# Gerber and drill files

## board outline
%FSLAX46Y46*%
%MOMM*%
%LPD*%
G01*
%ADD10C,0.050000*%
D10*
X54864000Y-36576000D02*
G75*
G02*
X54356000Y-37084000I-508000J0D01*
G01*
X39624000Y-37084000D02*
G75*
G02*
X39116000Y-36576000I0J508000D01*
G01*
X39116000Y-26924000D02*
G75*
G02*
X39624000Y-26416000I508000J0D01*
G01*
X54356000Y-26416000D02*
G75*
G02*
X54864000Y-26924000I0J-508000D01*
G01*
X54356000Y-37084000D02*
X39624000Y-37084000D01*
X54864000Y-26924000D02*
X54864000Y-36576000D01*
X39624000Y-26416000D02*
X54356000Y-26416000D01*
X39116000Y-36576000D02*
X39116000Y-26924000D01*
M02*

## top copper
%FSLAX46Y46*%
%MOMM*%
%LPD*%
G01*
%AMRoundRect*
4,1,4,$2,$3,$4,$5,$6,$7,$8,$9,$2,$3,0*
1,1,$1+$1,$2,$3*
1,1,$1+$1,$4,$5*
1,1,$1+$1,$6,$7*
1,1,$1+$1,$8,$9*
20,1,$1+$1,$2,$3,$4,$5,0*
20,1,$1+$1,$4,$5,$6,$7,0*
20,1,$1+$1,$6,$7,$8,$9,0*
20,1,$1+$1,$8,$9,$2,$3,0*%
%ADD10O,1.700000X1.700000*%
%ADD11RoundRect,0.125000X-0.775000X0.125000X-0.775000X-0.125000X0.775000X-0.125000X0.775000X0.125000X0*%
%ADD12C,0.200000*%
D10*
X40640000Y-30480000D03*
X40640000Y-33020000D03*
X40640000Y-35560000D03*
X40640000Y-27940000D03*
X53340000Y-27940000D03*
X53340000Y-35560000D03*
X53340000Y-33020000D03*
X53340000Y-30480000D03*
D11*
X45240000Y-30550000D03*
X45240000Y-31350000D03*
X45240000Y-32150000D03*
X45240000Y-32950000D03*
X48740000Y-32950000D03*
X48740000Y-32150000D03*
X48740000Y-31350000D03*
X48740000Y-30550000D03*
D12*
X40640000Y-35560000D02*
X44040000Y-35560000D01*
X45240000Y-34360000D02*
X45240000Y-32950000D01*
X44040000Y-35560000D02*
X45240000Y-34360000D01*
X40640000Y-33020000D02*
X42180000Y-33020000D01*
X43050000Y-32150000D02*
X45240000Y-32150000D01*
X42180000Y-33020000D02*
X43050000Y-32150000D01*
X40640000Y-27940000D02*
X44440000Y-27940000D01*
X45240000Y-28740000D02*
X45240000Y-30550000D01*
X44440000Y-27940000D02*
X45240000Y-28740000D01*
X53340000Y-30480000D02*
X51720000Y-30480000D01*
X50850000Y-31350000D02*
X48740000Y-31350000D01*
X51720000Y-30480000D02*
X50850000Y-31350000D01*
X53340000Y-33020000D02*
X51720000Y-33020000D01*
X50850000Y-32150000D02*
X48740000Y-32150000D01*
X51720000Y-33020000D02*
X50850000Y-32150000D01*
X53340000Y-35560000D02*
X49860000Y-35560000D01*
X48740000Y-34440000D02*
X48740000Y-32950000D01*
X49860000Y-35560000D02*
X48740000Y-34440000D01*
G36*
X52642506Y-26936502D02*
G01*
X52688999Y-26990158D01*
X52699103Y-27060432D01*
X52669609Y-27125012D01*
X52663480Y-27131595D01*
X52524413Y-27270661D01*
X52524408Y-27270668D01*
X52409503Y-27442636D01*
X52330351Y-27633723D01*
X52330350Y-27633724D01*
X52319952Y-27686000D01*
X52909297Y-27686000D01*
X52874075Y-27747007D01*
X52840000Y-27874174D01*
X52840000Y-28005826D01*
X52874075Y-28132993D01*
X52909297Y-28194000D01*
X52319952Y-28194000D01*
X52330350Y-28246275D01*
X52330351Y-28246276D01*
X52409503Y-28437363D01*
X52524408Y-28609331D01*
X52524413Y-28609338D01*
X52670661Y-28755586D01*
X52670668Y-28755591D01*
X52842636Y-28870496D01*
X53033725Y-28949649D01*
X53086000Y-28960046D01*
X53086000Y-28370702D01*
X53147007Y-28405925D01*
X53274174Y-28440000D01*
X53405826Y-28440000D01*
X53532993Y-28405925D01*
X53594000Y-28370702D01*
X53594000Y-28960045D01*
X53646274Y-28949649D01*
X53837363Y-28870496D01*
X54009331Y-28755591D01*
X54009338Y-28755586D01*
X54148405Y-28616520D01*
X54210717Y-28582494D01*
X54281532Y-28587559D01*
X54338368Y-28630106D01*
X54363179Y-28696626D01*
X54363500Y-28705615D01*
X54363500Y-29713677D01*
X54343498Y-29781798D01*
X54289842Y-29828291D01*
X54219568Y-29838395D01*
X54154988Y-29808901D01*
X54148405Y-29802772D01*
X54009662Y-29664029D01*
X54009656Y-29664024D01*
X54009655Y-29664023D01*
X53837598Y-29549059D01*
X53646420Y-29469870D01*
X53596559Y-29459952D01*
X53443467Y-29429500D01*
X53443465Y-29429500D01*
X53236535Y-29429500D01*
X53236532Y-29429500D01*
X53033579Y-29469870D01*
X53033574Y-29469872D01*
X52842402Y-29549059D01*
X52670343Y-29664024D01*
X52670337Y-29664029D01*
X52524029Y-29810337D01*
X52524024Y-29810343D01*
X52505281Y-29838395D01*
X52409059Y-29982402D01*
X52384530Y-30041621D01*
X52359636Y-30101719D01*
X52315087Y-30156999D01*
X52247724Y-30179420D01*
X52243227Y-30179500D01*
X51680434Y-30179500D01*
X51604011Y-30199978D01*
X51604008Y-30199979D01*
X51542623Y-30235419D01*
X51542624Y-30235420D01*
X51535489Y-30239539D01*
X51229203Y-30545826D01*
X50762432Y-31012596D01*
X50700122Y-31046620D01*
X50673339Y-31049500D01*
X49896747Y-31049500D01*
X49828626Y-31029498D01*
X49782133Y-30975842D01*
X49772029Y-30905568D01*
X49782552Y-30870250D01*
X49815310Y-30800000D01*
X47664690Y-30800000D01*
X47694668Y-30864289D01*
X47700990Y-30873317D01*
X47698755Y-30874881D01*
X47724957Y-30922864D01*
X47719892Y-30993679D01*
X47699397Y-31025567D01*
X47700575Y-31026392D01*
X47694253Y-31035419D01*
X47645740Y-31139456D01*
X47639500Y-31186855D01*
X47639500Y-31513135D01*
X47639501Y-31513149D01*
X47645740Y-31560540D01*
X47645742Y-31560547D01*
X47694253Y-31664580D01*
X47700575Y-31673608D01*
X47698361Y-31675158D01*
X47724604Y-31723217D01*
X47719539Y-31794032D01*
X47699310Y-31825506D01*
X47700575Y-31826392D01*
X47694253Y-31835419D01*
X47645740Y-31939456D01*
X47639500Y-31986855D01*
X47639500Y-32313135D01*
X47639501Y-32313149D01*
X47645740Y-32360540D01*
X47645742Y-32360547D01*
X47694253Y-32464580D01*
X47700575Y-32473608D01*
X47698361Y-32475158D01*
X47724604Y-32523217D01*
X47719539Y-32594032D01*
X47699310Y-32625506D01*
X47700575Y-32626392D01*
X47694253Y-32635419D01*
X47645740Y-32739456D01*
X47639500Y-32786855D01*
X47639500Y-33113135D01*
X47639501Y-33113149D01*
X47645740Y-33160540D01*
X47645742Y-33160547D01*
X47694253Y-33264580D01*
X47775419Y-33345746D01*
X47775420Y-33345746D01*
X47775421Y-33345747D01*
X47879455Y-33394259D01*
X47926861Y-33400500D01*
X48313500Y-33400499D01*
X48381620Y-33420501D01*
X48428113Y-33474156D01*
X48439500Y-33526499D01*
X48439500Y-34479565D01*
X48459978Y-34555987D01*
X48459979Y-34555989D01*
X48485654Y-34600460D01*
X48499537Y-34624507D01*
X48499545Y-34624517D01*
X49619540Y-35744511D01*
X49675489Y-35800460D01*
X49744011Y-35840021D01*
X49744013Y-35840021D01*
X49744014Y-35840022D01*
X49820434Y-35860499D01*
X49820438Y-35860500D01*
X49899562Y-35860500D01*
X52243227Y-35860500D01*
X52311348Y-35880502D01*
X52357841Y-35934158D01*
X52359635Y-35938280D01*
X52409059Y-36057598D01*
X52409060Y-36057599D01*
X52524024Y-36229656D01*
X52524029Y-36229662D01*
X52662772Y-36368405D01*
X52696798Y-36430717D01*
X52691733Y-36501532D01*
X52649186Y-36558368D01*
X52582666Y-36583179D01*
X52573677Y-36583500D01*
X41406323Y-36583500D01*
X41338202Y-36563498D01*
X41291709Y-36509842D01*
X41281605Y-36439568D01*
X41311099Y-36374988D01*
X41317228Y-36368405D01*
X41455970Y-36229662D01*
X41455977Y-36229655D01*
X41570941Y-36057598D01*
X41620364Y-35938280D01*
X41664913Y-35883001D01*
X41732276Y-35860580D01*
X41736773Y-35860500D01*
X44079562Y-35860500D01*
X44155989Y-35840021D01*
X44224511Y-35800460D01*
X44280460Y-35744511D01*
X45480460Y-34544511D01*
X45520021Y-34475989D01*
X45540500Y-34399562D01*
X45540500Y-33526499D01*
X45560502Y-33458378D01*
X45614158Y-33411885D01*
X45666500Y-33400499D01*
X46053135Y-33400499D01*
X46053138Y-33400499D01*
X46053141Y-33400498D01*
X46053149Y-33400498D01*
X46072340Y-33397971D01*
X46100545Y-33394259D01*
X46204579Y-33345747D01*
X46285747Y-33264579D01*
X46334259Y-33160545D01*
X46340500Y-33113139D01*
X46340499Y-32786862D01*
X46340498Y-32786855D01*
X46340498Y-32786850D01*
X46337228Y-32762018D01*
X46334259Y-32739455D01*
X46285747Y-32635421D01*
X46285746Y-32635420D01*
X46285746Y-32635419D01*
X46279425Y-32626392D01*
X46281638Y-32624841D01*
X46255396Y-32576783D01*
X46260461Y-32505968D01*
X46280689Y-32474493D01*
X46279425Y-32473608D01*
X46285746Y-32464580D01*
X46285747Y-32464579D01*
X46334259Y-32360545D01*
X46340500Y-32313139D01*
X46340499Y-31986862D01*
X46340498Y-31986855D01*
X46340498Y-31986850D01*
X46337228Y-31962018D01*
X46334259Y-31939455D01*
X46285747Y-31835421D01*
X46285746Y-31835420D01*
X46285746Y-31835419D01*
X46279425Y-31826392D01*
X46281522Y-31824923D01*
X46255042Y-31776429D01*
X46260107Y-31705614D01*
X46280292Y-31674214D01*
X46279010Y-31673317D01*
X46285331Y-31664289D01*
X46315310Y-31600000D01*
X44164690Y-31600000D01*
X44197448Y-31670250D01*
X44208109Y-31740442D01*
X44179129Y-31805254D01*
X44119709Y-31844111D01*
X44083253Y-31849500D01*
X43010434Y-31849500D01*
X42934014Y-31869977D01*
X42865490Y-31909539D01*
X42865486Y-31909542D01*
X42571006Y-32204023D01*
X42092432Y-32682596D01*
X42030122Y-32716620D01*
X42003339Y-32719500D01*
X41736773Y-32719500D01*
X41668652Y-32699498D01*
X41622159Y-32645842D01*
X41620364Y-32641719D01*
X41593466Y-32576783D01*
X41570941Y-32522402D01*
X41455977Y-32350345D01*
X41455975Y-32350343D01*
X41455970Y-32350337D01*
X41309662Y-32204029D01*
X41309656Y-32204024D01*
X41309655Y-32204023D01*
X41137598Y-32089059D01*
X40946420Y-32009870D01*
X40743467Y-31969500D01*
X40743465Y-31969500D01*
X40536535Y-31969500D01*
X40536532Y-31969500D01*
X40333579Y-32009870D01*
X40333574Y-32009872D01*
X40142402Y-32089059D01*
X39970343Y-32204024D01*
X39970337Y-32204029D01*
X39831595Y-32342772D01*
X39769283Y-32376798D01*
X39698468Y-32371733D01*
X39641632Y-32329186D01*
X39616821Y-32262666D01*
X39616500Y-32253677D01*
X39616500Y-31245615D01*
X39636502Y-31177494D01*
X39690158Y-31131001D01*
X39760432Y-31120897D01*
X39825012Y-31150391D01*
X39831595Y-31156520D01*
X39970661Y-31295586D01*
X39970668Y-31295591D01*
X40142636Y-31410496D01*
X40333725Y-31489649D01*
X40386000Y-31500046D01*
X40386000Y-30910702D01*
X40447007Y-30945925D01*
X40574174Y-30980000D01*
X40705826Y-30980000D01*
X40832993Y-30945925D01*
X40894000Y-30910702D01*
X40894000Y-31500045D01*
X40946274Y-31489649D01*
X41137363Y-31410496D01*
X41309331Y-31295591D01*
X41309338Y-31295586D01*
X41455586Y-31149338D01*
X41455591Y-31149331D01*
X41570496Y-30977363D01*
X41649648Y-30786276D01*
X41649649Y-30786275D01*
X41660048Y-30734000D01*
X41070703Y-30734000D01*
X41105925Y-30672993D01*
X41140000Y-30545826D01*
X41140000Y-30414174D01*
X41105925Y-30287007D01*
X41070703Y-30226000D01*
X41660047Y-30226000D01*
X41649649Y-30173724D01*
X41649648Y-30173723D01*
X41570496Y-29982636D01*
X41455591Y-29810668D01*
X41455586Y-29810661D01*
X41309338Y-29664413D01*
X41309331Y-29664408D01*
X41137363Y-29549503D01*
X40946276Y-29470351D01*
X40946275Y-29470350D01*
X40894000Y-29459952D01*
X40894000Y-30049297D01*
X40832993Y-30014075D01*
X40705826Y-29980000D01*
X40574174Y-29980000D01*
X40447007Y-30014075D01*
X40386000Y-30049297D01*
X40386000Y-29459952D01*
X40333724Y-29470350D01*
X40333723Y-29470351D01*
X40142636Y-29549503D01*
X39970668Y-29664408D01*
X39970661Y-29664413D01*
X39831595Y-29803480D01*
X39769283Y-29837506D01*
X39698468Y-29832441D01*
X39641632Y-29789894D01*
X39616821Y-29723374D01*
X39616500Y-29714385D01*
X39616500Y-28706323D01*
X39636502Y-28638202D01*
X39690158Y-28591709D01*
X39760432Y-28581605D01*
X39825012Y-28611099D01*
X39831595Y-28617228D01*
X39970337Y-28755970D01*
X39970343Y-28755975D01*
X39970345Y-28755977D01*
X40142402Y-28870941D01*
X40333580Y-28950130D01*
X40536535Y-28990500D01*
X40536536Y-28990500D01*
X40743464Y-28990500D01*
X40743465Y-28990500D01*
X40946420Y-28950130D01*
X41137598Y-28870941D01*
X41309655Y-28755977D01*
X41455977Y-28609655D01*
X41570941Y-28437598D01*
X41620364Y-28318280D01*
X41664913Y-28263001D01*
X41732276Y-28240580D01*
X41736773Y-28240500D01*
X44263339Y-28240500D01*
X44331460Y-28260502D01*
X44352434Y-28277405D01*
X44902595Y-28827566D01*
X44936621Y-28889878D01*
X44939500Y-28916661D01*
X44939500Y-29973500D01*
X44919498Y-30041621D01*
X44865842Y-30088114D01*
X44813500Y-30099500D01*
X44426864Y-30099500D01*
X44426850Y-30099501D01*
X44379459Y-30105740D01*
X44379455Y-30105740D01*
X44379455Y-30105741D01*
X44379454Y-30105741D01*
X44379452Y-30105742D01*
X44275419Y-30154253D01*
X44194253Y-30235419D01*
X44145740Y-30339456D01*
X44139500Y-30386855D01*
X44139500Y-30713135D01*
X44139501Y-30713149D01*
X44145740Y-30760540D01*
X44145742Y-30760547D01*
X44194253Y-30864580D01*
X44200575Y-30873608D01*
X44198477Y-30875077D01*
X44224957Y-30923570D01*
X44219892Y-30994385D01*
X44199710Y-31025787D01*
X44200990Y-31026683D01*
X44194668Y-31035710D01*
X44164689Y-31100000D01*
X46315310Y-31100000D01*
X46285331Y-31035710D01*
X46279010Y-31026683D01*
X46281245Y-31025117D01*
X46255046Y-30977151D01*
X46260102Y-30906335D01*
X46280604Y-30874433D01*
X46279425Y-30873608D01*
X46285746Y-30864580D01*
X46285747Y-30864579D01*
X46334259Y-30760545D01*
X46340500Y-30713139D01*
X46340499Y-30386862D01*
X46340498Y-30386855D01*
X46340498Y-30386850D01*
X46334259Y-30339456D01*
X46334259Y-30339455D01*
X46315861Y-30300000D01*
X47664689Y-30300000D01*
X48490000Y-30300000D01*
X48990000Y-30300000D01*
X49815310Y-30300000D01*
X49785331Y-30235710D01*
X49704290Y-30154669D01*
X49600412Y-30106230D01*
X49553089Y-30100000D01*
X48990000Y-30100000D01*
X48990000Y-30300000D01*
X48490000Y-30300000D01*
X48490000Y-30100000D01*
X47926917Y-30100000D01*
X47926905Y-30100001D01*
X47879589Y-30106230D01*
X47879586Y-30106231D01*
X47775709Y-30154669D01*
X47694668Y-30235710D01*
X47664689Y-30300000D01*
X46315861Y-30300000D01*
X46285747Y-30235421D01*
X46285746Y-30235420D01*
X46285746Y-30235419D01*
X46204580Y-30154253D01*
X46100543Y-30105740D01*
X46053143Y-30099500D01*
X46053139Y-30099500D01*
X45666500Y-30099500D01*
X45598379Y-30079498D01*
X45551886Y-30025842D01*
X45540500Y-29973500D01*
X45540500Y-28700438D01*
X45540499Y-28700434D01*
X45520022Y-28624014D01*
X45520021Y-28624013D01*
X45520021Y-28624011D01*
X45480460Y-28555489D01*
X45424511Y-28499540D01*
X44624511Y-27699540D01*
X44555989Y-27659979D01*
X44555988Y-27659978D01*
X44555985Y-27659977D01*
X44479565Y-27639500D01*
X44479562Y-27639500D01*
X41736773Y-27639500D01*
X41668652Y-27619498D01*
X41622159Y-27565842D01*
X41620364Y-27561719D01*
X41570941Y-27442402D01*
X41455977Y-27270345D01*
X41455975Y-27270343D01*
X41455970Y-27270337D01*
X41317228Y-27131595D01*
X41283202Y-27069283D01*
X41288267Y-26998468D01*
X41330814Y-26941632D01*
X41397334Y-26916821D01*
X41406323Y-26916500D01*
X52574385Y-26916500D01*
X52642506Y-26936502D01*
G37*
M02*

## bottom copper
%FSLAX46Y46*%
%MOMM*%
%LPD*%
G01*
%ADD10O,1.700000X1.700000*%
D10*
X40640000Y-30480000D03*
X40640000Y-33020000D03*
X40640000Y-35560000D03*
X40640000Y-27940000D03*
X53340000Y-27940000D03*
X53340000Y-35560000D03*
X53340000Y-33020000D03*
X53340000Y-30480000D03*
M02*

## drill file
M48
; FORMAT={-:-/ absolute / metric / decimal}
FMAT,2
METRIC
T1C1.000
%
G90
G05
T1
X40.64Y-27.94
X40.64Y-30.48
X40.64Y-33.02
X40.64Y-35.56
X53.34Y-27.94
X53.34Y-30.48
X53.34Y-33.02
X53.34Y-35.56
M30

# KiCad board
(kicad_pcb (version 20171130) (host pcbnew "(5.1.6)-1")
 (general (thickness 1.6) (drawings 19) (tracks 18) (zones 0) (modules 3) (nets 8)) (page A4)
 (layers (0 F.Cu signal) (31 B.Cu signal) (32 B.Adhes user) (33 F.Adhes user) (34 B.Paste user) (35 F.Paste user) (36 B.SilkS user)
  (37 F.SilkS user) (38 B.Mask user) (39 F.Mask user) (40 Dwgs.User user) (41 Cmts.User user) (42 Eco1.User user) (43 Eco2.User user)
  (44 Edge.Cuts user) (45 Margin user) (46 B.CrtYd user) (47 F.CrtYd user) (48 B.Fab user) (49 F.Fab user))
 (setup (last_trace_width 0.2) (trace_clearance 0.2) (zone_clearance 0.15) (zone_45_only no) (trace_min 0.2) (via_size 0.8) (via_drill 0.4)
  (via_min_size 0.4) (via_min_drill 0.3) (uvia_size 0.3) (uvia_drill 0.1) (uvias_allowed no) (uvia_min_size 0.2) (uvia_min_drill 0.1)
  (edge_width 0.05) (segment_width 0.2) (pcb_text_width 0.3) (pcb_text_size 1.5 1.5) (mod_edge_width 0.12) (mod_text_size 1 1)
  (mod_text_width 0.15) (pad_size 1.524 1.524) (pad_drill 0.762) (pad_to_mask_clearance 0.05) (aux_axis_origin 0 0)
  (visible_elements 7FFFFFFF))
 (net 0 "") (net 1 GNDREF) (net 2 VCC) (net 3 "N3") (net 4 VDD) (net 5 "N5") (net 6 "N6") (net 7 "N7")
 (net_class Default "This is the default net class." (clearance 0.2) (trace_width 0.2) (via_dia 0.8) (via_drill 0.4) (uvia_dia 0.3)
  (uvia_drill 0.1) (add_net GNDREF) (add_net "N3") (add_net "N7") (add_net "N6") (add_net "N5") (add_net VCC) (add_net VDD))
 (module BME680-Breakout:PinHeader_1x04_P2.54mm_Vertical (layer F.Cu) (at 40.64 31.75)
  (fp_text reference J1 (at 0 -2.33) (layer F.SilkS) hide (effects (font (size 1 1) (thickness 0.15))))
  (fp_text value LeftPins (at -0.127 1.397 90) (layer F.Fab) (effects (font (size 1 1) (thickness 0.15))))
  (pad 2 thru_hole oval (at 0 -1.27) (size 1.7 1.7) (drill 1) (layers *.Cu *.Mask) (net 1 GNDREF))
  (pad 3 thru_hole oval (at 0 1.27) (size 1.7 1.7) (drill 1) (layers *.Cu *.Mask) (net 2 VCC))
  (pad 4 thru_hole oval (at 0 3.81) (size 1.7 1.7) (drill 1) (layers *.Cu *.Mask) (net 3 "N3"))
  (pad 1 thru_hole oval (at 0 -3.81) (size 1.7 1.7) (drill 1) (layers *.Cu *.Mask) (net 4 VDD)))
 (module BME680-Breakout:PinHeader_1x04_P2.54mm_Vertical (layer F.Cu) (at 53.34 31.75)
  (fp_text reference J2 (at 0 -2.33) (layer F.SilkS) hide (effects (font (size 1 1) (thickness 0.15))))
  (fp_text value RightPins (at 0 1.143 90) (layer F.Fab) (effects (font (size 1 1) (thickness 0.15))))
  (pad 1 thru_hole oval (at 0 -3.81) (size 1.7 1.7) (drill 1) (layers *.Cu *.Mask) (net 1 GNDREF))
  (pad 4 thru_hole oval (at 0 3.81) (size 1.7 1.7) (drill 1) (layers *.Cu *.Mask) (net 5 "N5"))
  (pad 3 thru_hole oval (at 0 1.27) (size 1.7 1.7) (drill 1) (layers *.Cu *.Mask) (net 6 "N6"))
  (pad 2 thru_hole oval (at 0 -1.27) (size 1.7 1.7) (drill 1) (layers *.Cu *.Mask) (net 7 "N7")))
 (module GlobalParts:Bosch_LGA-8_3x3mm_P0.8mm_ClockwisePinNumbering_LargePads (layer F.Cu) (at 46.99 31.75)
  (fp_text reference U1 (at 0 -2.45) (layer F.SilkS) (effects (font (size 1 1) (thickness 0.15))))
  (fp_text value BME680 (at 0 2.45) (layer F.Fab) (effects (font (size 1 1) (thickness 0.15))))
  (pad 8 smd roundrect (at -1.75 -1.2 270) (size 0.5 1.8) (layers F.Cu F.Paste F.Mask) (roundrect_rratio 0.25) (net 4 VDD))
  (pad 7 smd roundrect (at -1.75 -0.4 270) (size 0.5 1.8) (layers F.Cu F.Paste F.Mask) (roundrect_rratio 0.25) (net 1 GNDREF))
  (pad 6 smd roundrect (at -1.75 0.4 270) (size 0.5 1.8) (layers F.Cu F.Paste F.Mask) (roundrect_rratio 0.25) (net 2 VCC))
  (pad 5 smd roundrect (at -1.75 1.2 270) (size 0.5 1.8) (layers F.Cu F.Paste F.Mask) (roundrect_rratio 0.25) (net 3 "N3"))
  (pad 4 smd roundrect (at 1.75 1.2 270) (size 0.5 1.8) (layers F.Cu F.Paste F.Mask) (roundrect_rratio 0.25) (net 5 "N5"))
  (pad 3 smd roundrect (at 1.75 0.4 270) (size 0.5 1.8) (layers F.Cu F.Paste F.Mask) (roundrect_rratio 0.25) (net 6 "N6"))
  (pad 2 smd roundrect (at 1.75 -0.4 270) (size 0.5 1.8) (layers F.Cu F.Paste F.Mask) (roundrect_rratio 0.25) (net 7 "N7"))
  (pad 1 smd roundrect (at 1.75 -1.2 270) (size 0.5 1.8) (layers F.Cu F.Paste F.Mask) (roundrect_rratio 0.25) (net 1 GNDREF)))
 (gr_arc (start 54.356 36.576) (end 54.356 37.084) (angle -90) (layer Edge.Cuts) (width 0.05))
 (gr_arc (start 39.624 36.576) (end 39.116 36.576) (angle -90) (layer Edge.Cuts) (width 0.05))
 (gr_arc (start 39.624 26.924) (end 39.624 26.416) (angle -90) (layer Edge.Cuts) (width 0.05))
 (gr_arc (start 54.356 26.924) (end 54.864 26.924) (angle -90) (layer Edge.Cuts) (width 0.05))
 (gr_line (start 54.356 37.084) (end 39.624 37.084) (layer Edge.Cuts) (width 0.05))
 (gr_line (start 54.864 26.924) (end 54.864 36.576) (layer Edge.Cuts) (width 0.05))
 (gr_line (start 39.624 26.416) (end 54.356 26.416) (layer Edge.Cuts) (width 0.05))
 (gr_line (start 39.116 36.576) (end 39.116 26.924) (layer Edge.Cuts) (width 0.05))
 (segment (start 40.64 35.56) (end 44.04 35.56) (width 0.2) (layer F.Cu) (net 3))
 (segment (start 45.24 34.36) (end 45.24 32.95) (width 0.2) (layer F.Cu) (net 3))
 (segment (start 44.04 35.56) (end 45.24 34.36) (width 0.2) (layer F.Cu) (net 3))
 (segment (start 40.64 33.02) (end 42.18 33.02) (width 0.2) (layer F.Cu) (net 2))
 (segment (start 43.05 32.15) (end 45.24 32.15) (width 0.2) (layer F.Cu) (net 2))
 (segment (start 42.18 33.02) (end 43.05 32.15) (width 0.2) (layer F.Cu) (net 2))
 (segment (start 40.64 27.94) (end 44.44 27.94) (width 0.2) (layer F.Cu) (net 4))
 (segment (start 45.24 28.74) (end 45.24 30.55) (width 0.2) (layer F.Cu) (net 4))
 (segment (start 44.44 27.94) (end 45.24 28.74) (width 0.2) (layer F.Cu) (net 4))
 (segment (start 53.34 30.48) (end 51.72 30.48) (width 0.2) (layer F.Cu) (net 7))
 (segment (start 50.85 31.35) (end 48.74 31.35) (width 0.2) (layer F.Cu) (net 7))
 (segment (start 51.72 30.48) (end 50.85 31.35) (width 0.2) (layer F.Cu) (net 7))
 (segment (start 53.34 33.02) (end 51.72 33.02) (width 0.2) (layer F.Cu) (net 6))
 (segment (start 50.85 32.15) (end 48.74 32.15) (width 0.2) (layer F.Cu) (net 6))
 (segment (start 51.72 33.02) (end 50.85 32.15) (width 0.2) (layer F.Cu) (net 6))
 (segment (start 53.34 35.56) (end 49.86 35.56) (width 0.2) (layer F.Cu) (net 5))
 (segment (start 48.74 34.44) (end 48.74 32.95) (width 0.2) (layer F.Cu) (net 5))
 (segment (start 49.86 35.56) (end 48.74 34.44) (width 0.2) (layer F.Cu) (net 5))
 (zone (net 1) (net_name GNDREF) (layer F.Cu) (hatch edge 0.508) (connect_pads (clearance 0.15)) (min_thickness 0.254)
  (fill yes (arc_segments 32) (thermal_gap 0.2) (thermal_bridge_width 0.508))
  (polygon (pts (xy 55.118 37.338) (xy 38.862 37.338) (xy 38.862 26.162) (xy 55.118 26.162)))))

